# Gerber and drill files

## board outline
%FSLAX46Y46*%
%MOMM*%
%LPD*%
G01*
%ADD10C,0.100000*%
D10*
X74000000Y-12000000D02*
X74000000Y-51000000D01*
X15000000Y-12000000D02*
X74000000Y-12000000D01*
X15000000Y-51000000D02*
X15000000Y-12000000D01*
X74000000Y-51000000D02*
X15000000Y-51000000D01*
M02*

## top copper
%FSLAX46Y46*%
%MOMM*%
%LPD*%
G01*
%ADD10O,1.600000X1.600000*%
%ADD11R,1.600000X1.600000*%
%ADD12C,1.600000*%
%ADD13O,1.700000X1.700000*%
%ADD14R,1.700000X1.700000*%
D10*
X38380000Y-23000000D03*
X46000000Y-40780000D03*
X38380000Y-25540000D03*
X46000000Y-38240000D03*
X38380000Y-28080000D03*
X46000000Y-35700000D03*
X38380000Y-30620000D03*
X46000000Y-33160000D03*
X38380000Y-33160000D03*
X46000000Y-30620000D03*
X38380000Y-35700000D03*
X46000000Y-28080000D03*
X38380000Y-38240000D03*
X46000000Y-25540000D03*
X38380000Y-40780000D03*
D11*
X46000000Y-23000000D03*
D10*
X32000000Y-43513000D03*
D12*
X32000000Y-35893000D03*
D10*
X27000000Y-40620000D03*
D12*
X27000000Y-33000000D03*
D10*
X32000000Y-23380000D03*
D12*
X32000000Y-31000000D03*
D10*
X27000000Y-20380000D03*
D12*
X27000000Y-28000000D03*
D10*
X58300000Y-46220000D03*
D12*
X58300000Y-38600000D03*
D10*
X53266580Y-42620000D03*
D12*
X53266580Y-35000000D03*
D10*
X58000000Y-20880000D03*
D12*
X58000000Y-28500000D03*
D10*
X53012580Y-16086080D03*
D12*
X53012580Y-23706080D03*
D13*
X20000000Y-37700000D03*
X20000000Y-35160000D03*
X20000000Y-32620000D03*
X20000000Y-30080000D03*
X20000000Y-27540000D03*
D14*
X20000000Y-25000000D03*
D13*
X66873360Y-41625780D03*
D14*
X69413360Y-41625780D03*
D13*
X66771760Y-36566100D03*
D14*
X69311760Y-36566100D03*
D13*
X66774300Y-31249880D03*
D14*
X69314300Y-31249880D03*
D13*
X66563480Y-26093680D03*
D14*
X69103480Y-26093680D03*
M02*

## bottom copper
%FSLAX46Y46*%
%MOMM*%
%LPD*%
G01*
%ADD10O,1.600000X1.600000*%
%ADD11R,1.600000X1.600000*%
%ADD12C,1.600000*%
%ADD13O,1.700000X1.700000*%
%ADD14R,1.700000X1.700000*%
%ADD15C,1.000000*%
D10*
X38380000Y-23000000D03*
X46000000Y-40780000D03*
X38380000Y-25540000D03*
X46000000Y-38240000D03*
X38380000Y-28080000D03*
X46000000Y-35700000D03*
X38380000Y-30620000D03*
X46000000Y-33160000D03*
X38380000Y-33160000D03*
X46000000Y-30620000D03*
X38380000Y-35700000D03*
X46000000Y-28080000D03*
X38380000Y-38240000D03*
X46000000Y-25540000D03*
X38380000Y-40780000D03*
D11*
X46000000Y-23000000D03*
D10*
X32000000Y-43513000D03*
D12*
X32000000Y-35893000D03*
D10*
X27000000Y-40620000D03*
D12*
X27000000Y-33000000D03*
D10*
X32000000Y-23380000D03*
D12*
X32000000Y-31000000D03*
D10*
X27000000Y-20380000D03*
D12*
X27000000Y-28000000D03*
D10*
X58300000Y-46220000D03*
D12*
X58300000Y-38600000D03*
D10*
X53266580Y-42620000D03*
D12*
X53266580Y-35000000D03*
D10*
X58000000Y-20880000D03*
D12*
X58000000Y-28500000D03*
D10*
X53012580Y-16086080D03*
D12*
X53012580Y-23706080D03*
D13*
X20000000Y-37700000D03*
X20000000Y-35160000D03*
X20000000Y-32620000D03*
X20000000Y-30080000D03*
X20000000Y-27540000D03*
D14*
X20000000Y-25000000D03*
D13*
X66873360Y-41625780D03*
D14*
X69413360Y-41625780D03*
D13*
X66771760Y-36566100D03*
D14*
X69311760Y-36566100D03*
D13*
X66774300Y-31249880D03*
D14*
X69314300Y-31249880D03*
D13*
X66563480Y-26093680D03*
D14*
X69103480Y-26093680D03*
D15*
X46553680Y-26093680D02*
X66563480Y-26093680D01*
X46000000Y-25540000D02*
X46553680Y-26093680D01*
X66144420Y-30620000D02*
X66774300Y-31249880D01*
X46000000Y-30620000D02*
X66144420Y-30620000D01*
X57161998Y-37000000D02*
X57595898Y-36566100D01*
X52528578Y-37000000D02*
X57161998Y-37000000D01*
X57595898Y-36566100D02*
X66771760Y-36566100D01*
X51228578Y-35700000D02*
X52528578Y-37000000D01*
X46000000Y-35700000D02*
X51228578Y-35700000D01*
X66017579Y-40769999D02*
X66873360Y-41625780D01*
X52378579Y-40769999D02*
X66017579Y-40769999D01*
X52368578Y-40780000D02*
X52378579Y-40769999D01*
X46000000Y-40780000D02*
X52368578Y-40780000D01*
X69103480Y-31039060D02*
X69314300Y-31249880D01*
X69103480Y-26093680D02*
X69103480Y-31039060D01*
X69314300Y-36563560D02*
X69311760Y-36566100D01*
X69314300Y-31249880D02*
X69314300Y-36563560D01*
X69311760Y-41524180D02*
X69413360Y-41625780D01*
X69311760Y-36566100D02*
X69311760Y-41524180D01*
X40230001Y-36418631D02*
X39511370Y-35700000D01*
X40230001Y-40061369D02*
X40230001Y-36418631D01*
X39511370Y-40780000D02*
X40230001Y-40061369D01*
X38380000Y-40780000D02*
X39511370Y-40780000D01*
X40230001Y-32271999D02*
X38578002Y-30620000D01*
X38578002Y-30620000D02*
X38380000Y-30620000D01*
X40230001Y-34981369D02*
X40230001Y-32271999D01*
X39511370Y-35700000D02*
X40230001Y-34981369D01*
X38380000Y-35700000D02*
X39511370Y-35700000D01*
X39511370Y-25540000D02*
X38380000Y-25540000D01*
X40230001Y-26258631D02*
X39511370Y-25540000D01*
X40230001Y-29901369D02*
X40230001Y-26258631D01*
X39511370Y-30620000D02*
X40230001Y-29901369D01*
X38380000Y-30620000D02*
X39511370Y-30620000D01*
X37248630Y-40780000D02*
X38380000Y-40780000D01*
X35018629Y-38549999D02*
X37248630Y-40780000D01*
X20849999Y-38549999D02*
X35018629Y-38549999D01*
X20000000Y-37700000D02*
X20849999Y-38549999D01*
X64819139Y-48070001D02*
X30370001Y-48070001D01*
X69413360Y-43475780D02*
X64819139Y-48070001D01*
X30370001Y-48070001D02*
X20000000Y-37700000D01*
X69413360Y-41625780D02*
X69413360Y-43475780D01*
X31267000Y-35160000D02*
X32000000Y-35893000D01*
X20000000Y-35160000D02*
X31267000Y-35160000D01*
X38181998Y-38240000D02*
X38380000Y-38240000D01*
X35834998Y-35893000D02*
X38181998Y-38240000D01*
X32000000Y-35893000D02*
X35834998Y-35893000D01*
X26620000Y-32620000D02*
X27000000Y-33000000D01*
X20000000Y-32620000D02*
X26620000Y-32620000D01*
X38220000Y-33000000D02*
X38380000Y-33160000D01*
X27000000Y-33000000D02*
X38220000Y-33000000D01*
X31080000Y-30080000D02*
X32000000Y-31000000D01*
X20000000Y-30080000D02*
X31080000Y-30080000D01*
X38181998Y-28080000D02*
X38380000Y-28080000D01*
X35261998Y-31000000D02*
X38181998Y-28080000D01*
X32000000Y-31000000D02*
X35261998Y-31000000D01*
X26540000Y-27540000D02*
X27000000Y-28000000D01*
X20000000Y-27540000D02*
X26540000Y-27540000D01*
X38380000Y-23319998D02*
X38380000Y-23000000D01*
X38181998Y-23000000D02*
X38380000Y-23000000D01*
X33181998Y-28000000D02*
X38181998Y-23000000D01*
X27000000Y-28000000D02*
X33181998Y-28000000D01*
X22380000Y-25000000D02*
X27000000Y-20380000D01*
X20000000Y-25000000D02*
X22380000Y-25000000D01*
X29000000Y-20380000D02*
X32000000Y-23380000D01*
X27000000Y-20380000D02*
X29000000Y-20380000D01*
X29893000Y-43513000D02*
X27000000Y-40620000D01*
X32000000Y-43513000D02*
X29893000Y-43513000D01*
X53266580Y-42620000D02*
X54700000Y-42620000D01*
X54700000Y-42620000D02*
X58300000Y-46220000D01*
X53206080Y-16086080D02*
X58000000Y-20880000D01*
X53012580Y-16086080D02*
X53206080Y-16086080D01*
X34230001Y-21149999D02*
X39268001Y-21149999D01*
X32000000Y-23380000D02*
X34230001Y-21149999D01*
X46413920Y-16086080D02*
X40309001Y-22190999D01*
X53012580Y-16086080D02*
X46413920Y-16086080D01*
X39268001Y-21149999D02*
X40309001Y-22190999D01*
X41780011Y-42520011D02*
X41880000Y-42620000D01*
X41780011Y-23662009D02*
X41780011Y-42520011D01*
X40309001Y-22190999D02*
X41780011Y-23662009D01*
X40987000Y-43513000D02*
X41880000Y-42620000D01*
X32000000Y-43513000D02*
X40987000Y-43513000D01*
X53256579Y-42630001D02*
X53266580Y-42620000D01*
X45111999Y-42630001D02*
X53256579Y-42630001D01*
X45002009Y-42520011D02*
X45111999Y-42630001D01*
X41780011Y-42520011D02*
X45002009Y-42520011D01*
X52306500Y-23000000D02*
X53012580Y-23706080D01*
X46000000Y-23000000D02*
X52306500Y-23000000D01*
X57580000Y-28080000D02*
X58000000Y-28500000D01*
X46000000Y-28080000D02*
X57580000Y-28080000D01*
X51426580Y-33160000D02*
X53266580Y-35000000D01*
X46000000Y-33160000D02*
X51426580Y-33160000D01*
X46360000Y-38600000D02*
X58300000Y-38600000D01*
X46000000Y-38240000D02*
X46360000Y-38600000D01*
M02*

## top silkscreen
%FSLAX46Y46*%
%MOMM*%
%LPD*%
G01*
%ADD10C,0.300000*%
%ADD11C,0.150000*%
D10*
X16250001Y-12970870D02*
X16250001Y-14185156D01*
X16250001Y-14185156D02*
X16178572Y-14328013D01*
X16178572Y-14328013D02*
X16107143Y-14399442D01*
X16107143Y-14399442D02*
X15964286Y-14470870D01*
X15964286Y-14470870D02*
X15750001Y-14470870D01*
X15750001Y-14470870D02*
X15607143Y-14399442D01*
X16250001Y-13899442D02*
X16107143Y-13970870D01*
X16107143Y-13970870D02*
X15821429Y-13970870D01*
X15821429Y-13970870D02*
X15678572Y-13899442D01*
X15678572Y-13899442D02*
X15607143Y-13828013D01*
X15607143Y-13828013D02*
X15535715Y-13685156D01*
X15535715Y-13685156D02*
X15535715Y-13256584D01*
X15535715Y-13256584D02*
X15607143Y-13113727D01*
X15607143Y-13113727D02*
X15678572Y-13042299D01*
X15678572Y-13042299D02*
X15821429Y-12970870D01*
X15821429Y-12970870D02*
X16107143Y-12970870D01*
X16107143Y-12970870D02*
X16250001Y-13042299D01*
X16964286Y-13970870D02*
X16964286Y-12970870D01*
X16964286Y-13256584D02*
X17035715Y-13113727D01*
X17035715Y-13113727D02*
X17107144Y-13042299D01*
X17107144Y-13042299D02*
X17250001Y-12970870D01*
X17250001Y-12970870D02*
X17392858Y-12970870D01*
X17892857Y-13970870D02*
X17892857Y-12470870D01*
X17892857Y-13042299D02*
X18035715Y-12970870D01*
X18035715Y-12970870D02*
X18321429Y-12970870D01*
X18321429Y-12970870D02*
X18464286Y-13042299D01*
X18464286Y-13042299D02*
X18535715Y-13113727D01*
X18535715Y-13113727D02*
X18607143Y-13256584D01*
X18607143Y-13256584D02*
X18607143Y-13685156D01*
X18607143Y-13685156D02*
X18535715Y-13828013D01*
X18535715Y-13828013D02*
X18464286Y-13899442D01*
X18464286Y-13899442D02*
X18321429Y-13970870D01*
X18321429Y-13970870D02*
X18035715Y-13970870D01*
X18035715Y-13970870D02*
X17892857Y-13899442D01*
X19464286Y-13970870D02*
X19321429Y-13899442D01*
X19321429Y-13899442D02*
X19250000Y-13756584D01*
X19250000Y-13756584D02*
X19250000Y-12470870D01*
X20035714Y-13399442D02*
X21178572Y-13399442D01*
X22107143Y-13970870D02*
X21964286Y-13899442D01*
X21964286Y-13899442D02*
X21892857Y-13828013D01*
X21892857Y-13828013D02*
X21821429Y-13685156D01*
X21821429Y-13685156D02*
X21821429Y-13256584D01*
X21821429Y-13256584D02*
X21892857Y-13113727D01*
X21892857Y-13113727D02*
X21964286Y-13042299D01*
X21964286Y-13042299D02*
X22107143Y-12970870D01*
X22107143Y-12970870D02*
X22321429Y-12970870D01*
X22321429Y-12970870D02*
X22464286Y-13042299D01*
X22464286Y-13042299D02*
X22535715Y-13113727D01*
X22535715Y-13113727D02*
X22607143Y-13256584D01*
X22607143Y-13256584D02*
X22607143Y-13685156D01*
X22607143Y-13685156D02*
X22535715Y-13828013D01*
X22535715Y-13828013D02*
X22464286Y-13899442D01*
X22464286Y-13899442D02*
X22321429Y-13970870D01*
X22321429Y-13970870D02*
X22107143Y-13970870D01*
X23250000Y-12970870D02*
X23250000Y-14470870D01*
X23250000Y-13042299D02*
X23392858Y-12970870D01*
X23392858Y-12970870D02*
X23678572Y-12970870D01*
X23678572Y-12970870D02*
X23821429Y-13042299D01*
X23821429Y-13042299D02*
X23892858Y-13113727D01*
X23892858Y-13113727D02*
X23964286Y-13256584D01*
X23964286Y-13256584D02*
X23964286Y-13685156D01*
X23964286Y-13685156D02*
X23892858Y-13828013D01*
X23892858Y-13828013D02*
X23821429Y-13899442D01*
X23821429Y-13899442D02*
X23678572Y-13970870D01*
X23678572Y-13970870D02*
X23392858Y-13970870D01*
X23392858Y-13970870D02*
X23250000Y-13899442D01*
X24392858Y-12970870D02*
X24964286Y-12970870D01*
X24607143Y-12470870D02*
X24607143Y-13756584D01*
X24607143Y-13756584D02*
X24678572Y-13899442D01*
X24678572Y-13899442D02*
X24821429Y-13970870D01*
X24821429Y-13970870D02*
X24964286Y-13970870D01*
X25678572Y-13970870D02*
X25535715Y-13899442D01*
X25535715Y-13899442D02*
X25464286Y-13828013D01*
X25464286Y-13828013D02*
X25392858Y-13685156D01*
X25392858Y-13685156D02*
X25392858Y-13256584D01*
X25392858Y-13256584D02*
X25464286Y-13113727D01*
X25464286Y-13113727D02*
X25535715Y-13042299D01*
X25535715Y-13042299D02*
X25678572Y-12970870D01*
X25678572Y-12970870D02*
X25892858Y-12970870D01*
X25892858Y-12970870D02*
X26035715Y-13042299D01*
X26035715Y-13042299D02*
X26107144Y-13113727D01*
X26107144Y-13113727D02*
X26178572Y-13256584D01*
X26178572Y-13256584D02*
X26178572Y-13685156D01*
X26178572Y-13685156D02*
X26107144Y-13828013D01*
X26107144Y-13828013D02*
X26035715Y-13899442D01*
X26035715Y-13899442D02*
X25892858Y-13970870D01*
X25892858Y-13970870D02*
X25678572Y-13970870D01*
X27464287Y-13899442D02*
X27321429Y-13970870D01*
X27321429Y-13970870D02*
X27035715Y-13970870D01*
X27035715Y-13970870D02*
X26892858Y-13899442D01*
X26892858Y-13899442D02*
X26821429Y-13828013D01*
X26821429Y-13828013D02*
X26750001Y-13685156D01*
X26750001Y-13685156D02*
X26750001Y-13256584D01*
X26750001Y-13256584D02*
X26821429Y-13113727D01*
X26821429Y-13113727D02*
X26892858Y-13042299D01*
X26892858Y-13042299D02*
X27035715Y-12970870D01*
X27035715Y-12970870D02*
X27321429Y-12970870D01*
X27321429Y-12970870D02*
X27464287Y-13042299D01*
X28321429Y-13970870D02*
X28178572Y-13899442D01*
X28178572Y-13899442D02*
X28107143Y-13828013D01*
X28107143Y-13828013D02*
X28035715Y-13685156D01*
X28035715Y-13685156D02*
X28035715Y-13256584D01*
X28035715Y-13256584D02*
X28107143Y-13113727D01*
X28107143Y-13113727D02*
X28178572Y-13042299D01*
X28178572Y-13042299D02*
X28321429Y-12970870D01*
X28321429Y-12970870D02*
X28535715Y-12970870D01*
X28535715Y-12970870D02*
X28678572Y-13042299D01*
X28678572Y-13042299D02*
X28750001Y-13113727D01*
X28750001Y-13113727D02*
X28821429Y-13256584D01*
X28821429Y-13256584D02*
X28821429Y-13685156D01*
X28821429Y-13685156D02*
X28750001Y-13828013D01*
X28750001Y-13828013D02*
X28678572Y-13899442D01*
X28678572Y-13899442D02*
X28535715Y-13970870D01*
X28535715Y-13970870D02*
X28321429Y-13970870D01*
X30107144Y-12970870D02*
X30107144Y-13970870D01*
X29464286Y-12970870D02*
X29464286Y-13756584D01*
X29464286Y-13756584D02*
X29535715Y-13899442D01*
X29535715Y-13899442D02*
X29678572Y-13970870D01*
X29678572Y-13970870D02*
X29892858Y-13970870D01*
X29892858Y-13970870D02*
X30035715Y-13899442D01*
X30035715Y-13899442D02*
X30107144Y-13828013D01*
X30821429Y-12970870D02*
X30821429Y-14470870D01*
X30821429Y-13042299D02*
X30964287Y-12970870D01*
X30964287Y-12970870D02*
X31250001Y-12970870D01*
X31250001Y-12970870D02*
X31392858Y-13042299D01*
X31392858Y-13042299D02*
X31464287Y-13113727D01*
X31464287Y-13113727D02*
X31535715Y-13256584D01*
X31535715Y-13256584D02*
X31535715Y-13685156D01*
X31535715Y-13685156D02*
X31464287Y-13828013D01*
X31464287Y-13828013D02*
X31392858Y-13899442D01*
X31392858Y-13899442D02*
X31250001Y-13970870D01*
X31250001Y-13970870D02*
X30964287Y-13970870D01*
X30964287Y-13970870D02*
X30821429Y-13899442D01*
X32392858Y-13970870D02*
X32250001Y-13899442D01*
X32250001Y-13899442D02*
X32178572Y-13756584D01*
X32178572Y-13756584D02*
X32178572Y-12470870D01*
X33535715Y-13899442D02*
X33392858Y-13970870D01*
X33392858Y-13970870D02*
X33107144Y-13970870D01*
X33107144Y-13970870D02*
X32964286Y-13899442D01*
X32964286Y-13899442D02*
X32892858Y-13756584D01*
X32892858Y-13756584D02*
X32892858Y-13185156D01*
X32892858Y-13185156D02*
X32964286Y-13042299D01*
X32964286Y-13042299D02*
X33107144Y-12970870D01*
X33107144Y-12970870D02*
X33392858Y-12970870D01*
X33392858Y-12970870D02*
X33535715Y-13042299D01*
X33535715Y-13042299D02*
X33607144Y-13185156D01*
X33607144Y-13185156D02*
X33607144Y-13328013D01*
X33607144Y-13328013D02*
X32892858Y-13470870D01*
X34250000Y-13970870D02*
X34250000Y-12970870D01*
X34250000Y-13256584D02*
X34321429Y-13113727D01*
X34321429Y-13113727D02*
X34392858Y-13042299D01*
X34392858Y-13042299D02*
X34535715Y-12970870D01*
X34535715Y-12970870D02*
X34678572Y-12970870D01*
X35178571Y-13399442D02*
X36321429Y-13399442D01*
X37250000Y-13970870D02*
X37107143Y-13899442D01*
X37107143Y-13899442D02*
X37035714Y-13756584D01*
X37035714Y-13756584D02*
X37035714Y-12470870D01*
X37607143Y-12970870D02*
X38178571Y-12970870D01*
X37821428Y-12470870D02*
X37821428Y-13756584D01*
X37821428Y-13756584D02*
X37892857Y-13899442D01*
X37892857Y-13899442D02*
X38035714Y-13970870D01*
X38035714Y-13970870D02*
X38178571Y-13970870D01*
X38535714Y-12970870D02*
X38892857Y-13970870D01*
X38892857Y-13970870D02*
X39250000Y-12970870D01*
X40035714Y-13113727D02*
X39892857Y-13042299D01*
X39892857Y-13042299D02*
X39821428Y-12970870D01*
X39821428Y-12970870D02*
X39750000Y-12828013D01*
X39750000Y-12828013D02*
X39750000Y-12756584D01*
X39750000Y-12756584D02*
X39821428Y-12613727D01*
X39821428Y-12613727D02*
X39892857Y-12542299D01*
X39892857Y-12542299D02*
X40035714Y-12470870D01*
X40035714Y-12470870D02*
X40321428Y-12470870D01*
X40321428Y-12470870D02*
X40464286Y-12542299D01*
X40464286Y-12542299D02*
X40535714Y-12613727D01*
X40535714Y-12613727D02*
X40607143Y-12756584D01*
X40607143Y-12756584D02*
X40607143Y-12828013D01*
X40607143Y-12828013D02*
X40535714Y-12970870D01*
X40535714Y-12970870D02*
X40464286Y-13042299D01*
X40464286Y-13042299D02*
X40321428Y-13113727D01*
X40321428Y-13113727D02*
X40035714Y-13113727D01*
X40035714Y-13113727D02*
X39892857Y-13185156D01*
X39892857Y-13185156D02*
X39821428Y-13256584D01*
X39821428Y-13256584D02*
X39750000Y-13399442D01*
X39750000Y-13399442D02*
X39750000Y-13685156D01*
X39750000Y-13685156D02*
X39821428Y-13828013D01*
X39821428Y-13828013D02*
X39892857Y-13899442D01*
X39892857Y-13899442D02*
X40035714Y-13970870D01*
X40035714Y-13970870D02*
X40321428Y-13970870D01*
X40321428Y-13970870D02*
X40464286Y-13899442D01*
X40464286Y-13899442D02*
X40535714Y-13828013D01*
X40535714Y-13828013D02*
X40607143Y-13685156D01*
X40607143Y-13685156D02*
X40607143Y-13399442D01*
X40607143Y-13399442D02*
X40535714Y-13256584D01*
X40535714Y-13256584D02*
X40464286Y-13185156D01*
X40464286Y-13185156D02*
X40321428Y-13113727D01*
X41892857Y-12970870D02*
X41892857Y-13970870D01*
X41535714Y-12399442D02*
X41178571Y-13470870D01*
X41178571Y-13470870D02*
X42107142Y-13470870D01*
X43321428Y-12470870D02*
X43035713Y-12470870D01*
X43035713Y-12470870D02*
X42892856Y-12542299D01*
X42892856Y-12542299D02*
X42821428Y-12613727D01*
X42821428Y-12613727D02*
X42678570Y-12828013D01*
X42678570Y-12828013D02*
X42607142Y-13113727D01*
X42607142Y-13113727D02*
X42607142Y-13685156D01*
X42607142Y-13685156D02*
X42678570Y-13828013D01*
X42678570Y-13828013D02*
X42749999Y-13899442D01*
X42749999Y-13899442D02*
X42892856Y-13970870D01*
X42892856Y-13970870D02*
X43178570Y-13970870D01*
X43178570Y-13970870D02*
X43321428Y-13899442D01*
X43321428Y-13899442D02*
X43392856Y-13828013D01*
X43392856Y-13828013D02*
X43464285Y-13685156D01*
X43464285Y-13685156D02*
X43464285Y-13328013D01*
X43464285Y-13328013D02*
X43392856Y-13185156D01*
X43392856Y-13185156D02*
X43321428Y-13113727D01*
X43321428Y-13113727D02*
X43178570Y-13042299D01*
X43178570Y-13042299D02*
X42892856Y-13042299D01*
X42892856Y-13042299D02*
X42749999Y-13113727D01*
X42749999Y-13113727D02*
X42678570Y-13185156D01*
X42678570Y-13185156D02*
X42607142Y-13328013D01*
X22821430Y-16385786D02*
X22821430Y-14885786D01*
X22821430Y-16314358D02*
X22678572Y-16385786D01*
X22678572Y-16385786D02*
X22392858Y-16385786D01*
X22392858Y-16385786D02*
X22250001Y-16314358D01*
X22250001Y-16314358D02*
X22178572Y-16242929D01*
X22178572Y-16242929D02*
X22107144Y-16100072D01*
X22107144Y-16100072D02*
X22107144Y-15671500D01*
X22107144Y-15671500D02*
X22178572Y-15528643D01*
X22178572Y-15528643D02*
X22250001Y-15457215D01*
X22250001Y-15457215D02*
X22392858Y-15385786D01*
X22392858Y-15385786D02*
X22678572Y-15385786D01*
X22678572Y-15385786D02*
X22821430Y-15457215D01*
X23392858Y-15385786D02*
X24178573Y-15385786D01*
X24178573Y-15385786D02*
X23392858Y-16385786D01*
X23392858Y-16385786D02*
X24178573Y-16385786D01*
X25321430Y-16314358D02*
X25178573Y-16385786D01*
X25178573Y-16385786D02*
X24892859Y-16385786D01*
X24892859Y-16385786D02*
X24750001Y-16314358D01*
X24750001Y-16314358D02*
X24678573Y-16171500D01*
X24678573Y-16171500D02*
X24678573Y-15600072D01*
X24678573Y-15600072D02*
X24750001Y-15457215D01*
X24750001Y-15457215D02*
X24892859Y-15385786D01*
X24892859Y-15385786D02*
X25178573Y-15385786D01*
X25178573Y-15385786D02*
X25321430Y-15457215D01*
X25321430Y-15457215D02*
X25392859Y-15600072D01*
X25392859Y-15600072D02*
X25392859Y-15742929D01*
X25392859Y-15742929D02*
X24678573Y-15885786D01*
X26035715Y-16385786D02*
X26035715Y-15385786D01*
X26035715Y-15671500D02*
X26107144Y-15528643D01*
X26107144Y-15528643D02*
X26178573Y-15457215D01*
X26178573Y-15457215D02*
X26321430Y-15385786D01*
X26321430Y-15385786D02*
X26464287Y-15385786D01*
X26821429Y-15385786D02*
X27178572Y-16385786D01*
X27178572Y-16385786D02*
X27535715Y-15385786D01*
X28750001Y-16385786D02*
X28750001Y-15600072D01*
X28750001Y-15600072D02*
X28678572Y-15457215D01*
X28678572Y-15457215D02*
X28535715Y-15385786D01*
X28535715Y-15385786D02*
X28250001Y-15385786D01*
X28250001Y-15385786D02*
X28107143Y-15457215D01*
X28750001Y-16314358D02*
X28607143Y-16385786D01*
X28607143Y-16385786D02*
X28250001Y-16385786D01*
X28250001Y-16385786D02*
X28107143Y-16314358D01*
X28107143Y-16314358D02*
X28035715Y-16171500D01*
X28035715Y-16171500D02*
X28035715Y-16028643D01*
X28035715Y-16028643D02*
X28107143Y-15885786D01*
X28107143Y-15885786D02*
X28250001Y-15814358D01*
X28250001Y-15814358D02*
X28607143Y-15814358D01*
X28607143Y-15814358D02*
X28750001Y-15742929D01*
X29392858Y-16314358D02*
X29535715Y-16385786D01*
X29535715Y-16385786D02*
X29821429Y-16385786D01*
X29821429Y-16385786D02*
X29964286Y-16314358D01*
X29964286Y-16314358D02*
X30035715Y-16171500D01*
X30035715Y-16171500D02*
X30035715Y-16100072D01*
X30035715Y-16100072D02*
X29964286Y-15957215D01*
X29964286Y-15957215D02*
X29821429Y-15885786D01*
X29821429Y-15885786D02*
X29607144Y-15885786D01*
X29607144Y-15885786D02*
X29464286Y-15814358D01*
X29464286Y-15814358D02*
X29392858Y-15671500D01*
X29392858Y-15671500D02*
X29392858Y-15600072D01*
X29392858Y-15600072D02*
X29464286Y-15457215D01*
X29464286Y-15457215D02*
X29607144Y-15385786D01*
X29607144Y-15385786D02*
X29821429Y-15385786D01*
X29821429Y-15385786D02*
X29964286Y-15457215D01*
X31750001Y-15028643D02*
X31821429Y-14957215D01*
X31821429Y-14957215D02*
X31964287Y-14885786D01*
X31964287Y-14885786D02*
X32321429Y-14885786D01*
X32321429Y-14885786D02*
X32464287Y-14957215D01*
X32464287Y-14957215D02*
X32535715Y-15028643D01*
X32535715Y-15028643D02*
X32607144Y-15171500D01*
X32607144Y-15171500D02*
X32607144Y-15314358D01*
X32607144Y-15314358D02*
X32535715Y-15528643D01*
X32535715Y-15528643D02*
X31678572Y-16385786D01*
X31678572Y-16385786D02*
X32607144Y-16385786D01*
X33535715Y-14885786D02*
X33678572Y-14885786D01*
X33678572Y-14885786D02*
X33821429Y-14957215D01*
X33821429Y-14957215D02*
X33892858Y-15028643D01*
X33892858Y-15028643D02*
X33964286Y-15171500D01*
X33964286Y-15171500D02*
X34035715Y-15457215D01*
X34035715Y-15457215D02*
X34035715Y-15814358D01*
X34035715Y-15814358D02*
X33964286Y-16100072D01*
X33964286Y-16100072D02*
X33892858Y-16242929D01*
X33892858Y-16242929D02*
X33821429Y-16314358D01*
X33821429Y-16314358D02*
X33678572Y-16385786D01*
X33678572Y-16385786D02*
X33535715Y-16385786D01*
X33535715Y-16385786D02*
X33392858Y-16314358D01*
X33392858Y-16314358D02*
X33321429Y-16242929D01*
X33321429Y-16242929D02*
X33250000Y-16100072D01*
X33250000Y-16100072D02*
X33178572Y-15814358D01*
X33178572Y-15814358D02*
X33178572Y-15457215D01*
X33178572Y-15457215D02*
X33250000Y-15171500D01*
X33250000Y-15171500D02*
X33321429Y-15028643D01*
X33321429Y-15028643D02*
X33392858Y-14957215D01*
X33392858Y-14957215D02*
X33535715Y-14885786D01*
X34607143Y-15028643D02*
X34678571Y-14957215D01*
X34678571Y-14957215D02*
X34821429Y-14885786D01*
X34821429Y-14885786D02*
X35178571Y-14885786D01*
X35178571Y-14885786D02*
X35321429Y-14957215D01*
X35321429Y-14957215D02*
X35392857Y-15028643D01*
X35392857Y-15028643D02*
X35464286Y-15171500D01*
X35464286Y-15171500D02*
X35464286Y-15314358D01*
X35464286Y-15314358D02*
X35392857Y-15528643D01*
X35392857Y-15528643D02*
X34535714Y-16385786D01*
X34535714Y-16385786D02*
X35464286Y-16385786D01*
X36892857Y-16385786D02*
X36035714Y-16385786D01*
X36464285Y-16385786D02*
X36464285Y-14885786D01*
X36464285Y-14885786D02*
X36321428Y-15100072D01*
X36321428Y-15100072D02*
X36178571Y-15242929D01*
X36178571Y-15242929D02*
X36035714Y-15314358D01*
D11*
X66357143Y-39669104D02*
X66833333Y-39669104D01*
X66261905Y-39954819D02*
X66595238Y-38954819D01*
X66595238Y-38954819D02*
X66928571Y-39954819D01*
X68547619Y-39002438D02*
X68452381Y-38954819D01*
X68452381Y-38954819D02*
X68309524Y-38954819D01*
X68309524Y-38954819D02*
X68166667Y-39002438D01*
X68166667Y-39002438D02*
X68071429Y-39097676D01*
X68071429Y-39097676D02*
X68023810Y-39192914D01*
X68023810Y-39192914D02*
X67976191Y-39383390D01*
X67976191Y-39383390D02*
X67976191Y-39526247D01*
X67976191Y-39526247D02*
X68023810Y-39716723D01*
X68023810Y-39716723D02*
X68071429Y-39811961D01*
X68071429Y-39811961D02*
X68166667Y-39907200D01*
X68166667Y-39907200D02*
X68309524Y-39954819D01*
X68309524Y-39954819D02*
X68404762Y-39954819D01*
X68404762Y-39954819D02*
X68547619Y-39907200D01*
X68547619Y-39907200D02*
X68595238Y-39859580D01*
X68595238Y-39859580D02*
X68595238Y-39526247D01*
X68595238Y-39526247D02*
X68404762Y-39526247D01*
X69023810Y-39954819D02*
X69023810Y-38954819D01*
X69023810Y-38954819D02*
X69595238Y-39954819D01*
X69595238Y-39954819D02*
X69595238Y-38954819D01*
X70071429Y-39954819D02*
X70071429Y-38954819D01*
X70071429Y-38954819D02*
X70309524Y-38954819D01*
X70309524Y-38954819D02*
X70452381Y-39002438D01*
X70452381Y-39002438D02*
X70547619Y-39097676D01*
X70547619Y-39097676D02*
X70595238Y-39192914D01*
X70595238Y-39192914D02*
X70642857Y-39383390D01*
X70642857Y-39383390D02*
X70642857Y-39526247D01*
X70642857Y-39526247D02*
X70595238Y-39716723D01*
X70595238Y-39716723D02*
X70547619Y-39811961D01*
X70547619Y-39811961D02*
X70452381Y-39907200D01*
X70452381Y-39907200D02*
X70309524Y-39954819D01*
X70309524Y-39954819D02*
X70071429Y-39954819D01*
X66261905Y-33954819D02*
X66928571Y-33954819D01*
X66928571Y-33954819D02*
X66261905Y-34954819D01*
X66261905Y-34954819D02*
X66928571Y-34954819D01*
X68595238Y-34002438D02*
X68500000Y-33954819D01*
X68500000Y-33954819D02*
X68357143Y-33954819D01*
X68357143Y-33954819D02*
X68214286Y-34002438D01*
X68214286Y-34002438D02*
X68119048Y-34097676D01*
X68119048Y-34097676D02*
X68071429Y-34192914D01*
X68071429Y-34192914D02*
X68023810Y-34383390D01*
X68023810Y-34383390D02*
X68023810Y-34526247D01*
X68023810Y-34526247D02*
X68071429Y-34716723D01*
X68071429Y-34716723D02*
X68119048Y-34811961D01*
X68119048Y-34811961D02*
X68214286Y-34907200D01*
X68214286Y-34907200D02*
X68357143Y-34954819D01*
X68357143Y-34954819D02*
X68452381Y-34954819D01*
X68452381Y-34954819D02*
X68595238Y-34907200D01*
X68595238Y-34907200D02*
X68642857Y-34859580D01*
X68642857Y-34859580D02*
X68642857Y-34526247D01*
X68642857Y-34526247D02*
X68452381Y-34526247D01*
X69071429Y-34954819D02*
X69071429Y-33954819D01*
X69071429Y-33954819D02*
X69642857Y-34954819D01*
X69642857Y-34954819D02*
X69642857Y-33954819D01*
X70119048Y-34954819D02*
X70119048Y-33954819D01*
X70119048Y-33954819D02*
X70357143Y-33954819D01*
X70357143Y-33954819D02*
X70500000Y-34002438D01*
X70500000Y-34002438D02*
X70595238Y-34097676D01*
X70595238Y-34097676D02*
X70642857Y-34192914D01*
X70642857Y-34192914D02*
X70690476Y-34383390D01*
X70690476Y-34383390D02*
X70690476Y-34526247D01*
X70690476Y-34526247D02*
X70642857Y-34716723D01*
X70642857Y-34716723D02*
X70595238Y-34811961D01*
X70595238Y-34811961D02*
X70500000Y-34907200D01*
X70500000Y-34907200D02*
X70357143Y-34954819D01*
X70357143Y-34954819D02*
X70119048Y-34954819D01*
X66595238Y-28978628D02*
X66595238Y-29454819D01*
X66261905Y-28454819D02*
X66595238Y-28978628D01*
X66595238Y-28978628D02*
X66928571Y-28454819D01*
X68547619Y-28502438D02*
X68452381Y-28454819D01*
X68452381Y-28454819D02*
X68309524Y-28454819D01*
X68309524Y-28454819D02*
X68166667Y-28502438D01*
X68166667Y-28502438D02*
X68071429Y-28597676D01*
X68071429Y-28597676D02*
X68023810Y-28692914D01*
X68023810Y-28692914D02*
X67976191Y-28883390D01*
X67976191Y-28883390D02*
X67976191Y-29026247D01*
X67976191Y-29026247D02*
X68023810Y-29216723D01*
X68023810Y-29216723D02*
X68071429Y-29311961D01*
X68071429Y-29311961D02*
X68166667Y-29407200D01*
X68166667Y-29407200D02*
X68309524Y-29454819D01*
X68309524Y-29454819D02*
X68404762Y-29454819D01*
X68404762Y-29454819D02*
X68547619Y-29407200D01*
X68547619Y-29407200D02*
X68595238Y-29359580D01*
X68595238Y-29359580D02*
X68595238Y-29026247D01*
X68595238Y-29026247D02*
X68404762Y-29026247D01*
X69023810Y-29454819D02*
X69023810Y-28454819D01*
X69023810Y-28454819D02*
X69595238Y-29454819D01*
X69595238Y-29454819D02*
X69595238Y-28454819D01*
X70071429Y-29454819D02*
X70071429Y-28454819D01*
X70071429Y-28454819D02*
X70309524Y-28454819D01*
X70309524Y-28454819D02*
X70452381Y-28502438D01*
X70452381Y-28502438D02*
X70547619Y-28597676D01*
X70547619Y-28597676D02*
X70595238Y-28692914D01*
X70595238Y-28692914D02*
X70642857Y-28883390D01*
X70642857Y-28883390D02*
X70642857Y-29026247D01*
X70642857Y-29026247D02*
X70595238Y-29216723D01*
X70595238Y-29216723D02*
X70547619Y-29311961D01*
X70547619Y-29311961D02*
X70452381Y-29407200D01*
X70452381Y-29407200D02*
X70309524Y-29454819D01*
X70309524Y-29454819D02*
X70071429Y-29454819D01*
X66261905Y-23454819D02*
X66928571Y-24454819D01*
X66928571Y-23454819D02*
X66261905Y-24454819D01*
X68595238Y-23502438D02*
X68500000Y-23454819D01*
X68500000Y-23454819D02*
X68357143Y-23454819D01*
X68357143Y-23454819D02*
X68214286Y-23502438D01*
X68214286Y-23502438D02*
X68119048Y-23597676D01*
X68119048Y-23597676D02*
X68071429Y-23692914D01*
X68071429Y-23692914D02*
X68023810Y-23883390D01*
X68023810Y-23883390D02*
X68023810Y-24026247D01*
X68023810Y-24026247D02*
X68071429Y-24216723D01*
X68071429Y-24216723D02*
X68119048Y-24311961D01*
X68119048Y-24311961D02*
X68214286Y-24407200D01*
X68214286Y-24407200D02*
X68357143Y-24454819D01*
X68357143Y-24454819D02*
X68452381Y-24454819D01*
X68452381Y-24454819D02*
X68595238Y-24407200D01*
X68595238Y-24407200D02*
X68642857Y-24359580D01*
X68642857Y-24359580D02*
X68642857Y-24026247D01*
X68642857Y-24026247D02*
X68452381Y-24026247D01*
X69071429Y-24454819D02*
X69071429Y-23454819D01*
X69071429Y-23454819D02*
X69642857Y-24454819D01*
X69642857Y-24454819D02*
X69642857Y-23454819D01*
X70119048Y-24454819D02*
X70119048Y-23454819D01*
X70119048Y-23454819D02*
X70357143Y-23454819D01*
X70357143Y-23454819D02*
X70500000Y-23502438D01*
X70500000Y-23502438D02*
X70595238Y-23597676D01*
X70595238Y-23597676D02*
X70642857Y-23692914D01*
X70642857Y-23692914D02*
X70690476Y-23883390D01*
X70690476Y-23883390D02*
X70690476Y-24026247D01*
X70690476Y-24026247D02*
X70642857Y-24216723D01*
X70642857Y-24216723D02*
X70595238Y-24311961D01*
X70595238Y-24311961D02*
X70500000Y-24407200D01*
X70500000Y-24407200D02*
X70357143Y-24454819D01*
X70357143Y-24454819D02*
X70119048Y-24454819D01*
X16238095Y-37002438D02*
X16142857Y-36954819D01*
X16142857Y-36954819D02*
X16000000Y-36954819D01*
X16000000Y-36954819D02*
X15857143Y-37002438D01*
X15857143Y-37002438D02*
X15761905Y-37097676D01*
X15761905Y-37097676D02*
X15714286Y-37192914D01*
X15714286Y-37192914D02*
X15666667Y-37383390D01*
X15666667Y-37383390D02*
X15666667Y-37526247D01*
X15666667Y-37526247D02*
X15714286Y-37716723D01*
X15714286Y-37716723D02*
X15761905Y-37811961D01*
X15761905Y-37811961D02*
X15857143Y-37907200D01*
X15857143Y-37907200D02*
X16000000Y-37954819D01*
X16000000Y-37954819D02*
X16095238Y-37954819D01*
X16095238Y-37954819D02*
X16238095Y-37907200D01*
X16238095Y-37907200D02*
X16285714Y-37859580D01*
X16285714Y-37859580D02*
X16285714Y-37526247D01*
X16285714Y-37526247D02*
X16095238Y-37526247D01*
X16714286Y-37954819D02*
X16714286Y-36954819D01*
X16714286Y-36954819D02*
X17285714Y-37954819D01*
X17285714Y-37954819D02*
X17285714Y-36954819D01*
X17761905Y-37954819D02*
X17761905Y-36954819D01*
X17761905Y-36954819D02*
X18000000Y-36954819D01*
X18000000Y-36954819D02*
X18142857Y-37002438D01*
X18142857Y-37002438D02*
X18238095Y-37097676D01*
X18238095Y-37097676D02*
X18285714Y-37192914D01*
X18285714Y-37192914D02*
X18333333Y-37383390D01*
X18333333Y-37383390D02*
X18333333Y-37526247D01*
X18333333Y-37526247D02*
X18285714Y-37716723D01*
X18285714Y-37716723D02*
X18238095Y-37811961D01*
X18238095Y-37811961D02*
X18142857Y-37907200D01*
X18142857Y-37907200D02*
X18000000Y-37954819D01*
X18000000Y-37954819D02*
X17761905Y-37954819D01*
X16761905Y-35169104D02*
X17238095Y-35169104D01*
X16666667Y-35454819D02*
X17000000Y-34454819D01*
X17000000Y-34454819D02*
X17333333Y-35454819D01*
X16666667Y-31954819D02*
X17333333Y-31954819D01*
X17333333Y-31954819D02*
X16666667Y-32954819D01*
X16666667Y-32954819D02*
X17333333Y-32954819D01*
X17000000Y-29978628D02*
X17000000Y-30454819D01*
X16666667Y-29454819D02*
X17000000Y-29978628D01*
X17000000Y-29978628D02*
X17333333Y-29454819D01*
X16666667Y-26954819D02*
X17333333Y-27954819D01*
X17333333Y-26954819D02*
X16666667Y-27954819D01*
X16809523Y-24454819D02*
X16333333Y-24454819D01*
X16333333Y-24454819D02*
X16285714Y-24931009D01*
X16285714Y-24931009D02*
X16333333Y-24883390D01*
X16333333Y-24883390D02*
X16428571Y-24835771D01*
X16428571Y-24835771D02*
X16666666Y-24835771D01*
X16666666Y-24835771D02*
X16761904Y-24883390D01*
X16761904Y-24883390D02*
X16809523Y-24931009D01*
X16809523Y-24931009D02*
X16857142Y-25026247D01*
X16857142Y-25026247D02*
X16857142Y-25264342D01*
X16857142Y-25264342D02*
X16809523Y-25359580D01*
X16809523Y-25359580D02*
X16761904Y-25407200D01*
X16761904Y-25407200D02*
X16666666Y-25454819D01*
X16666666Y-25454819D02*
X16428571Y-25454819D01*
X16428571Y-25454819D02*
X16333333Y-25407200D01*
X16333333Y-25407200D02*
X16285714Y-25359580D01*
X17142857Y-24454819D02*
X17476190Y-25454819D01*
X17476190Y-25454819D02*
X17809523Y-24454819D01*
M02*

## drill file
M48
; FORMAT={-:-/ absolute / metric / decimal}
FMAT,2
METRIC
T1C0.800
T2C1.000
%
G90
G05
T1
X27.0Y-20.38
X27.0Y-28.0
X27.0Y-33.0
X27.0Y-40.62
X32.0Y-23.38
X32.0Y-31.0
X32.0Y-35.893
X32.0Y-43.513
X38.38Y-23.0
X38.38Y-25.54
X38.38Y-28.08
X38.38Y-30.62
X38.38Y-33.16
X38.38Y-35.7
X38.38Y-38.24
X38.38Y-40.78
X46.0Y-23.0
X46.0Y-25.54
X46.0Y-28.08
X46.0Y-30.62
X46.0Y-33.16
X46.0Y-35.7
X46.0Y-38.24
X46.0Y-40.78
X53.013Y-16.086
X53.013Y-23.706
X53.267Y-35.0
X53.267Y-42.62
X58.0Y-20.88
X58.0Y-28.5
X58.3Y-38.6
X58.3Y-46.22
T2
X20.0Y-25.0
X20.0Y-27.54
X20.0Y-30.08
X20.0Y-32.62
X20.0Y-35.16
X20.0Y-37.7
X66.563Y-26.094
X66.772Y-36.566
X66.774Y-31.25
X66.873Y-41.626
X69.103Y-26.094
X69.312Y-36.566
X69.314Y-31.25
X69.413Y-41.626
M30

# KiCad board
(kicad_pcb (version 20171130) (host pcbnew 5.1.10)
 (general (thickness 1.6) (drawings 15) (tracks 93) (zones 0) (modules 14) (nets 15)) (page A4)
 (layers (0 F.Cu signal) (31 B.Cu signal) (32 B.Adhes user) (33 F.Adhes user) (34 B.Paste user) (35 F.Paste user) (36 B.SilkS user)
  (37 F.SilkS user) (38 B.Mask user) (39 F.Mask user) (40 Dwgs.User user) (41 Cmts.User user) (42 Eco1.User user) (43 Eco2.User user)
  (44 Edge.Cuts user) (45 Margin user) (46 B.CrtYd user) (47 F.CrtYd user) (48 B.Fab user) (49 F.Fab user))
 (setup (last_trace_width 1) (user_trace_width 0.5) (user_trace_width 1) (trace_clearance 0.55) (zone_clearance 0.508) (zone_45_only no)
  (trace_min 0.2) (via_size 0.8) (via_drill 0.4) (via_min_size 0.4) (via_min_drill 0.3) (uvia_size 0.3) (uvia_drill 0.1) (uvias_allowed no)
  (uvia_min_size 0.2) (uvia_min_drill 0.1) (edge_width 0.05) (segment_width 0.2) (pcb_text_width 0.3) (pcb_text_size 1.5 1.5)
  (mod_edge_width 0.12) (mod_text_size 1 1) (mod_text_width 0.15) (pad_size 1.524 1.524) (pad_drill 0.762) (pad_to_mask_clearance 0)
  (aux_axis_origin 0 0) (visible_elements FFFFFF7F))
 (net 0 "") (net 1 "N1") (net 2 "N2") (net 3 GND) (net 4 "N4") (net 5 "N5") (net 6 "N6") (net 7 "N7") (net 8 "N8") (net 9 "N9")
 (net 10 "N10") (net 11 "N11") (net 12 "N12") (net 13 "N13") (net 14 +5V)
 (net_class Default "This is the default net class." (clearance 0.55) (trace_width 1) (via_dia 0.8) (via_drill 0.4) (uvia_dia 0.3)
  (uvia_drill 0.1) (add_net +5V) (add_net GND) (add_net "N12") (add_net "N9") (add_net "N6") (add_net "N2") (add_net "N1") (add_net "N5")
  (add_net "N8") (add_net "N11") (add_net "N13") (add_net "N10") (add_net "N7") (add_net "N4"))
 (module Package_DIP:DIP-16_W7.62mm (layer B.Cu) (at 46 23 180)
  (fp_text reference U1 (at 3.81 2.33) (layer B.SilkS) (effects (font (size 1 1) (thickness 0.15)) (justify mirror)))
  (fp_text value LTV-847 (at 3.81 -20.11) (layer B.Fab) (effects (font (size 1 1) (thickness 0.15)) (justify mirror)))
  (pad 16 thru_hole oval (at 7.62 0 180) (size 1.6 1.6) (drill 0.8) (layers *.Cu *.Mask) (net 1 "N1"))
  (pad 8 thru_hole oval (at 0 -17.78 180) (size 1.6 1.6) (drill 0.8) (layers *.Cu *.Mask) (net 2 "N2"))
  (pad 15 thru_hole oval (at 7.62 -2.54 180) (size 1.6 1.6) (drill 0.8) (layers *.Cu *.Mask) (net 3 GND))
  (pad 7 thru_hole oval (at 0 -15.24 180) (size 1.6 1.6) (drill 0.8) (layers *.Cu *.Mask) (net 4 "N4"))
  (pad 14 thru_hole oval (at 7.62 -5.08 180) (size 1.6 1.6) (drill 0.8) (layers *.Cu *.Mask) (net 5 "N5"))
  (pad 6 thru_hole oval (at 0 -12.7 180) (size 1.6 1.6) (drill 0.8) (layers *.Cu *.Mask) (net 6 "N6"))
  (pad 13 thru_hole oval (at 7.62 -7.62 180) (size 1.6 1.6) (drill 0.8) (layers *.Cu *.Mask) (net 3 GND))
  (pad 5 thru_hole oval (at 0 -10.16 180) (size 1.6 1.6) (drill 0.8) (layers *.Cu *.Mask) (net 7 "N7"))
  (pad 12 thru_hole oval (at 7.62 -10.16 180) (size 1.6 1.6) (drill 0.8) (layers *.Cu *.Mask) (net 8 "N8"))
  (pad 4 thru_hole oval (at 0 -7.62 180) (size 1.6 1.6) (drill 0.8) (layers *.Cu *.Mask) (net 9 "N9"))
  (pad 11 thru_hole oval (at 7.62 -12.7 180) (size 1.6 1.6) (drill 0.8) (layers *.Cu *.Mask) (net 3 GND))
  (pad 3 thru_hole oval (at 0 -5.08 180) (size 1.6 1.6) (drill 0.8) (layers *.Cu *.Mask) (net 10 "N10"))
  (pad 10 thru_hole oval (at 7.62 -15.24 180) (size 1.6 1.6) (drill 0.8) (layers *.Cu *.Mask) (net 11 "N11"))
  (pad 2 thru_hole oval (at 0 -2.54 180) (size 1.6 1.6) (drill 0.8) (layers *.Cu *.Mask) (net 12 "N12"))
  (pad 9 thru_hole oval (at 7.62 -17.78 180) (size 1.6 1.6) (drill 0.8) (layers *.Cu *.Mask) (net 3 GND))
  (pad 1 thru_hole rect (at 0 0 180) (size 1.6 1.6) (drill 0.8) (layers *.Cu *.Mask) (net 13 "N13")))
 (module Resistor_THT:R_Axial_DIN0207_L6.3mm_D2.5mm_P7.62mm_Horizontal (layer B.Cu) (at 32 35.893 270)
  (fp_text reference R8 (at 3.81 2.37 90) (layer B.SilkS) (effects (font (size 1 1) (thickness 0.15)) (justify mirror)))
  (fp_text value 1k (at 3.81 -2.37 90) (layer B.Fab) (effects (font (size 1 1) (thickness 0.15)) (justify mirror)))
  (pad 2 thru_hole oval (at 7.62 0 270) (size 1.6 1.6) (drill 0.8) (layers *.Cu *.Mask) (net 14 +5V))
  (pad 1 thru_hole circle (at 0 0 270) (size 1.6 1.6) (drill 0.8) (layers *.Cu *.Mask) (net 11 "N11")))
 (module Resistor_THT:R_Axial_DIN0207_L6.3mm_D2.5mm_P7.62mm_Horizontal (layer B.Cu) (at 27 33 270)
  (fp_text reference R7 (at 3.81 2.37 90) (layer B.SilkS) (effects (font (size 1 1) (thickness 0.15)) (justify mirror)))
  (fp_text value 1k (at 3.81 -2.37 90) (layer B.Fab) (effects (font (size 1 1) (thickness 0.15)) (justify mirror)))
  (pad 2 thru_hole oval (at 7.62 0 270) (size 1.6 1.6) (drill 0.8) (layers *.Cu *.Mask) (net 14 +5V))
  (pad 1 thru_hole circle (at 0 0 270) (size 1.6 1.6) (drill 0.8) (layers *.Cu *.Mask) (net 8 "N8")))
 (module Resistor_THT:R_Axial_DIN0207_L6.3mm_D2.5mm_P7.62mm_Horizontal (layer B.Cu) (at 32 31 90)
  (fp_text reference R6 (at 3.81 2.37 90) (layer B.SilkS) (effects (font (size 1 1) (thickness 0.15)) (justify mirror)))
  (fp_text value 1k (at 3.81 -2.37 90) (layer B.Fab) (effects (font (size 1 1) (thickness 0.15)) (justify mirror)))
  (pad 2 thru_hole oval (at 7.62 0 90) (size 1.6 1.6) (drill 0.8) (layers *.Cu *.Mask) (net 14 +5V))
  (pad 1 thru_hole circle (at 0 0 90) (size 1.6 1.6) (drill 0.8) (layers *.Cu *.Mask) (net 5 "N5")))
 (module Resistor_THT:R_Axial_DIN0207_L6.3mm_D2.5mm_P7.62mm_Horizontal (layer B.Cu) (at 27 28 90)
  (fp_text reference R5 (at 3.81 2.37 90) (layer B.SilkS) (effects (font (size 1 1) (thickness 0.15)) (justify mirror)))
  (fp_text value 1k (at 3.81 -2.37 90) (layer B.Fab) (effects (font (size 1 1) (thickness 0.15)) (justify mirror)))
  (pad 2 thru_hole oval (at 7.62 0 90) (size 1.6 1.6) (drill 0.8) (layers *.Cu *.Mask) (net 14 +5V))
  (pad 1 thru_hole circle (at 0 0 90) (size 1.6 1.6) (drill 0.8) (layers *.Cu *.Mask) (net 1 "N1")))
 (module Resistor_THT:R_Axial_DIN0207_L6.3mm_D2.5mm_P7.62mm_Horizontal (layer B.Cu) (at 58.3 38.6 270)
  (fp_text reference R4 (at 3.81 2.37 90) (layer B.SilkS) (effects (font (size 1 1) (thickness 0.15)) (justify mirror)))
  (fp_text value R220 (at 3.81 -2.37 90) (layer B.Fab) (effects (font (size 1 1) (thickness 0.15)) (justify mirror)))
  (pad 2 thru_hole oval (at 7.62 0 270) (size 1.6 1.6) (drill 0.8) (layers *.Cu *.Mask) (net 14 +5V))
  (pad 1 thru_hole circle (at 0 0 270) (size 1.6 1.6) (drill 0.8) (layers *.Cu *.Mask) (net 4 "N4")))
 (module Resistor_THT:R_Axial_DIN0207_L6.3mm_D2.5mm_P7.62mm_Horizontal (layer B.Cu) (at 53.26658 35 270)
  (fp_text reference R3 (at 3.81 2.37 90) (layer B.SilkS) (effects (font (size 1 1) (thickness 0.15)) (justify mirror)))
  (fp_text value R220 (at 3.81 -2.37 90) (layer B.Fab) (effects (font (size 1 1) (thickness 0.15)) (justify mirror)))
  (pad 2 thru_hole oval (at 7.62 0 270) (size 1.6 1.6) (drill 0.8) (layers *.Cu *.Mask) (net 14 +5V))
  (pad 1 thru_hole circle (at 0 0 270) (size 1.6 1.6) (drill 0.8) (layers *.Cu *.Mask) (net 7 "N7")))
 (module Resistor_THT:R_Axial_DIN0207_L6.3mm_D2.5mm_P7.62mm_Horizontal (layer B.Cu) (at 58 28.5 90)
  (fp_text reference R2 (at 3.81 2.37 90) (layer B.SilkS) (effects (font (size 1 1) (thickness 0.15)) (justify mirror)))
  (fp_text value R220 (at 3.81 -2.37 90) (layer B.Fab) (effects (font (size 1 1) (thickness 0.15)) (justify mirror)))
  (pad 2 thru_hole oval (at 7.62 0 90) (size 1.6 1.6) (drill 0.8) (layers *.Cu *.Mask) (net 14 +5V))
  (pad 1 thru_hole circle (at 0 0 90) (size 1.6 1.6) (drill 0.8) (layers *.Cu *.Mask) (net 10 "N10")))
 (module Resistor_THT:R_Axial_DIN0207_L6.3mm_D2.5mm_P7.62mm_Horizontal (layer B.Cu) (at 53.01258 23.70608 90)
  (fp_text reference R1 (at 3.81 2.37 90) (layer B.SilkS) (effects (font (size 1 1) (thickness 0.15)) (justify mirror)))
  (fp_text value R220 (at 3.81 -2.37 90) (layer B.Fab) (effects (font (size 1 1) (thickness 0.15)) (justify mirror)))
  (pad 2 thru_hole oval (at 7.62 0 90) (size 1.6 1.6) (drill 0.8) (layers *.Cu *.Mask) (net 14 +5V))
  (pad 1 thru_hole circle (at 0 0 90) (size 1.6 1.6) (drill 0.8) (layers *.Cu *.Mask) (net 13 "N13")))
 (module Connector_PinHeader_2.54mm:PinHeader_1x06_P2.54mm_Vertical (layer B.Cu) (at 20 25 180)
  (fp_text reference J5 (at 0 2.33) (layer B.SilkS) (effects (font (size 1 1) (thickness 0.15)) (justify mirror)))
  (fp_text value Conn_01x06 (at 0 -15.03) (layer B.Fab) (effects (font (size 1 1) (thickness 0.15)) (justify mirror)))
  (pad 6 thru_hole oval (at 0 -12.7 180) (size 1.7 1.7) (drill 1) (layers *.Cu *.Mask) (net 3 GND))
  (pad 5 thru_hole oval (at 0 -10.16 180) (size 1.7 1.7) (drill 1) (layers *.Cu *.Mask) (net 11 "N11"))
  (pad 4 thru_hole oval (at 0 -7.62 180) (size 1.7 1.7) (drill 1) (layers *.Cu *.Mask) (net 8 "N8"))
  (pad 3 thru_hole oval (at 0 -5.08 180) (size 1.7 1.7) (drill 1) (layers *.Cu *.Mask) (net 5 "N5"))
  (pad 2 thru_hole oval (at 0 -2.54 180) (size 1.7 1.7) (drill 1) (layers *.Cu *.Mask) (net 1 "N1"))
  (pad 1 thru_hole rect (at 0 0 180) (size 1.7 1.7) (drill 1) (layers *.Cu *.Mask) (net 14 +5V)))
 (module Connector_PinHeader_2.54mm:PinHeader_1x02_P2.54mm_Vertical (layer B.Cu) (at 69.41336 41.62578 90)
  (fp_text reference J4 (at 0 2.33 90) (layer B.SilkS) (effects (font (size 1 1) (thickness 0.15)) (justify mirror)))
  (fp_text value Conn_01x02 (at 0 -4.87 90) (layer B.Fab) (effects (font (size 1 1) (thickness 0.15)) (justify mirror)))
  (pad 2 thru_hole oval (at 0 -2.54 90) (size 1.7 1.7) (drill 1) (layers *.Cu *.Mask) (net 2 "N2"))
  (pad 1 thru_hole rect (at 0 0 90) (size 1.7 1.7) (drill 1) (layers *.Cu *.Mask) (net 3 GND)))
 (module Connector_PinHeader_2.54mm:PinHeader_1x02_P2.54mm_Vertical (layer B.Cu) (at 69.31176 36.5661 90)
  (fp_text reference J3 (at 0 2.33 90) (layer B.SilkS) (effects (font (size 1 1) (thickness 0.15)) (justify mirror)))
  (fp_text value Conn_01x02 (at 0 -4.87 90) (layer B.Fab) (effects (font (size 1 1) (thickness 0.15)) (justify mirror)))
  (pad 2 thru_hole oval (at 0 -2.54 90) (size 1.7 1.7) (drill 1) (layers *.Cu *.Mask) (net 6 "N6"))
  (pad 1 thru_hole rect (at 0 0 90) (size 1.7 1.7) (drill 1) (layers *.Cu *.Mask) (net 3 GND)))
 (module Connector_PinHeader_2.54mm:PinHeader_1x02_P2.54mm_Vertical (layer B.Cu) (at 69.3143 31.24988 90)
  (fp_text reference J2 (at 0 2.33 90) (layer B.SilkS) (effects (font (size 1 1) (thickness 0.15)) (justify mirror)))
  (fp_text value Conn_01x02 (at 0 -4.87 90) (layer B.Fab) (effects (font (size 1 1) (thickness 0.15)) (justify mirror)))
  (pad 2 thru_hole oval (at 0 -2.54 90) (size 1.7 1.7) (drill 1) (layers *.Cu *.Mask) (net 9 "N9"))
  (pad 1 thru_hole rect (at 0 0 90) (size 1.7 1.7) (drill 1) (layers *.Cu *.Mask) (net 3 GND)))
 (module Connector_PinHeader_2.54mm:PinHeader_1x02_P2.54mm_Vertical (layer B.Cu) (at 69.10348 26.09368 90)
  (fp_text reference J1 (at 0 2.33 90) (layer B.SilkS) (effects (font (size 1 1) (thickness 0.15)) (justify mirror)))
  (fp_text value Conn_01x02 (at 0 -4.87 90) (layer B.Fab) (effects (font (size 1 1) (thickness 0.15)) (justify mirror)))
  (pad 2 thru_hole oval (at 0 -2.54 90) (size 1.7 1.7) (drill 1) (layers *.Cu *.Mask) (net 12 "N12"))
  (pad 1 thru_hole rect (at 0 0 90) (size 1.7 1.7) (drill 1) (layers *.Cu *.Mask) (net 3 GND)))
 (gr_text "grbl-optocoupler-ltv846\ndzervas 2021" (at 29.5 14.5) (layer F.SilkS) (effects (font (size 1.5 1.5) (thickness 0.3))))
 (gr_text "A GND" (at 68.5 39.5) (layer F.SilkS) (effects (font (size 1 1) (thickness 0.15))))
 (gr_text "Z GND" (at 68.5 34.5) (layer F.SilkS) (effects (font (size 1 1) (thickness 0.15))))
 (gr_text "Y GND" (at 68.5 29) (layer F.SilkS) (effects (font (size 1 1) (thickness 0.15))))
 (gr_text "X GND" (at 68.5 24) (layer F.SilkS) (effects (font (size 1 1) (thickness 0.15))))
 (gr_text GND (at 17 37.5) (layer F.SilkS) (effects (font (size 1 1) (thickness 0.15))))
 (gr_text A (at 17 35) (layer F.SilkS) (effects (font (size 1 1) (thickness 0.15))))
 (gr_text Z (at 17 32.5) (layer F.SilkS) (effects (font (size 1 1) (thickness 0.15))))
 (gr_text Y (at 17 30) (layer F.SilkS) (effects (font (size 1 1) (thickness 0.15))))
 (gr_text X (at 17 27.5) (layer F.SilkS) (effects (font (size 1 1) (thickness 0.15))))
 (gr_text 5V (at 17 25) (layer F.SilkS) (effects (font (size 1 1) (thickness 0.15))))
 (gr_line (start 74 12) (end 74 51) (layer Edge.Cuts) (width 0.1))
 (gr_line (start 15 12) (end 74 12) (layer Edge.Cuts) (width 0.1))
 (gr_line (start 15 51) (end 15 12) (layer Edge.Cuts) (width 0.1))
 (gr_line (start 74 51) (end 15 51) (layer Edge.Cuts) (width 0.1))
 (segment (start 46.55368 26.09368) (end 66.56348 26.09368) (width 1) (layer B.Cu) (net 12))
 (segment (start 46 25.54) (end 46.55368 26.09368) (width 1) (layer B.Cu) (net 12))
 (segment (start 66.14442 30.62) (end 66.7743 31.24988) (width 1) (layer B.Cu) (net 9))
 (segment (start 46 30.62) (end 66.14442 30.62) (width 1) (layer B.Cu) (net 9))
 (segment (start 57.161998 37) (end 57.595898 36.5661) (width 1) (layer B.Cu) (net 6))
 (segment (start 52.528578 37) (end 57.161998 37) (width 1) (layer B.Cu) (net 6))
 (segment (start 57.595898 36.5661) (end 66.77176 36.5661) (width 1) (layer B.Cu) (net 6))
 (segment (start 51.228578 35.7) (end 52.528578 37) (width 1) (layer B.Cu) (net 6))
 (segment (start 46 35.7) (end 51.228578 35.7) (width 1) (layer B.Cu) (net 6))
 (segment (start 66.017579 40.769999) (end 66.87336 41.62578) (width 1) (layer B.Cu) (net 2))
 (segment (start 52.378579 40.769999) (end 66.017579 40.769999) (width 1) (layer B.Cu) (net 2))
 (segment (start 52.368578 40.78) (end 52.378579 40.769999) (width 1) (layer B.Cu) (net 2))
 (segment (start 46 40.78) (end 52.368578 40.78) (width 1) (layer B.Cu) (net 2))
 (segment (start 69.10348 31.03906) (end 69.3143 31.24988) (width 1) (layer B.Cu) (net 3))
 (segment (start 69.10348 26.09368) (end 69.10348 31.03906) (width 1) (layer B.Cu) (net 3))
 (segment (start 69.3143 36.56356) (end 69.31176 36.5661) (width 1) (layer B.Cu) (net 3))
 (segment (start 69.3143 31.24988) (end 69.3143 36.56356) (width 1) (layer B.Cu) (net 3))
 (segment (start 69.31176 41.52418) (end 69.41336 41.62578) (width 1) (layer B.Cu) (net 3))
 (segment (start 69.31176 36.5661) (end 69.31176 41.52418) (width 1) (layer B.Cu) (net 3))
 (segment (start 40.230001 36.418631) (end 39.51137 35.7) (width 1) (layer B.Cu) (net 3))
 (segment (start 40.230001 40.061369) (end 40.230001 36.418631) (width 1) (layer B.Cu) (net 3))
 (segment (start 39.51137 40.78) (end 40.230001 40.061369) (width 1) (layer B.Cu) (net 3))
 (segment (start 38.38 40.78) (end 39.51137 40.78) (width 1) (layer B.Cu) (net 3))
 (segment (start 40.230001 32.271999) (end 38.578002 30.62) (width 1) (layer B.Cu) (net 3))
 (segment (start 38.578002 30.62) (end 38.38 30.62) (width 1) (layer B.Cu) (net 3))
 (segment (start 40.230001 34.981369) (end 40.230001 32.271999) (width 1) (layer B.Cu) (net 3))
 (segment (start 39.51137 35.7) (end 40.230001 34.981369) (width 1) (layer B.Cu) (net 3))
 (segment (start 38.38 35.7) (end 39.51137 35.7) (width 1) (layer B.Cu) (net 3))
 (segment (start 39.51137 25.54) (end 38.38 25.54) (width 1) (layer B.Cu) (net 3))
 (segment (start 40.230001 26.258631) (end 39.51137 25.54) (width 1) (layer B.Cu) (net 3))
 (segment (start 40.230001 29.901369) (end 40.230001 26.258631) (width 1) (layer B.Cu) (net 3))
 (segment (start 39.51137 30.62) (end 40.230001 29.901369) (width 1) (layer B.Cu) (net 3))
 (segment (start 38.38 30.62) (end 39.51137 30.62) (width 1) (layer B.Cu) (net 3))
 (segment (start 37.24863 40.78) (end 38.38 40.78) (width 1) (layer B.Cu) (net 3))
 (segment (start 35.018629 38.549999) (end 37.24863 40.78) (width 1) (layer B.Cu) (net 3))
 (segment (start 20.849999 38.549999) (end 35.018629 38.549999) (width 1) (layer B.Cu) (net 3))
 (segment (start 20 37.7) (end 20.849999 38.549999) (width 1) (layer B.Cu) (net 3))
 (segment (start 64.819139 48.070001) (end 30.370001 48.070001) (width 1) (layer B.Cu) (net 3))
 (segment (start 69.41336 43.47578) (end 64.819139 48.070001) (width 1) (layer B.Cu) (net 3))
 (segment (start 30.370001 48.070001) (end 20 37.7) (width 1) (layer B.Cu) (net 3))
 (segment (start 69.41336 41.62578) (end 69.41336 43.47578) (width 1) (layer B.Cu) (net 3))
 (segment (start 31.267 35.16) (end 32 35.893) (width 1) (layer B.Cu) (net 11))
 (segment (start 20 35.16) (end 31.267 35.16) (width 1) (layer B.Cu) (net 11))
 (segment (start 38.181998 38.24) (end 38.38 38.24) (width 1) (layer B.Cu) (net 11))
 (segment (start 35.834998 35.893) (end 38.181998 38.24) (width 1) (layer B.Cu) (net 11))
 (segment (start 32 35.893) (end 35.834998 35.893) (width 1) (layer B.Cu) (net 11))
 (segment (start 26.62 32.62) (end 27 33) (width 1) (layer B.Cu) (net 8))
 (segment (start 20 32.62) (end 26.62 32.62) (width 1) (layer B.Cu) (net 8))
 (segment (start 38.22 33) (end 38.38 33.16) (width 1) (layer B.Cu) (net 8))
 (segment (start 27 33) (end 38.22 33) (width 1) (layer B.Cu) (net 8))
 (segment (start 31.08 30.08) (end 32 31) (width 1) (layer B.Cu) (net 5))
 (segment (start 20 30.08) (end 31.08 30.08) (width 1) (layer B.Cu) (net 5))
 (segment (start 38.181998 28.08) (end 38.38 28.08) (width 1) (layer B.Cu) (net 5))
 (segment (start 35.261998 31) (end 38.181998 28.08) (width 1) (layer B.Cu) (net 5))
 (segment (start 32 31) (end 35.261998 31) (width 1) (layer B.Cu) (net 5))
 (segment (start 26.54 27.54) (end 27 28) (width 1) (layer B.Cu) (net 1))
 (segment (start 20 27.54) (end 26.54 27.54) (width 1) (layer B.Cu) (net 1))
 (segment (start 38.38 23.319998) (end 38.38 23) (width 1) (layer B.Cu) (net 1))
 (segment (start 38.181998 23) (end 38.38 23) (width 1) (layer B.Cu) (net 1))
 (segment (start 33.181998 28) (end 38.181998 23) (width 1) (layer B.Cu) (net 1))
 (segment (start 27 28) (end 33.181998 28) (width 1) (layer B.Cu) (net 1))
 (segment (start 22.38 25) (end 27 20.38) (width 1) (layer B.Cu) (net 14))
 (segment (start 20 25) (end 22.38 25) (width 1) (layer B.Cu) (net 14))
 (segment (start 29 20.38) (end 32 23.38) (width 1) (layer B.Cu) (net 14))
 (segment (start 27 20.38) (end 29 20.38) (width 1) (layer B.Cu) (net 14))
 (segment (start 29.893 43.513) (end 27 40.62) (width 1) (layer B.Cu) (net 14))
 (segment (start 32 43.513) (end 29.893 43.513) (width 1) (layer B.Cu) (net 14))
 (segment (start 53.26658 42.62) (end 54.7 42.62) (width 1) (layer B.Cu) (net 14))
 (segment (start 54.7 42.62) (end 58.3 46.22) (width 1) (layer B.Cu) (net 14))
 (segment (start 53.20608 16.08608) (end 58 20.88) (width 1) (layer B.Cu) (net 14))
 (segment (start 53.01258 16.08608) (end 53.20608 16.08608) (width 1) (layer B.Cu) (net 14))
 (segment (start 34.230001 21.149999) (end 39.268001 21.149999) (width 1) (layer B.Cu) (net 14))
 (segment (start 32 23.38) (end 34.230001 21.149999) (width 1) (layer B.Cu) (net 14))
 (segment (start 46.41392 16.08608) (end 40.309001 22.190999) (width 1) (layer B.Cu) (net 14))
 (segment (start 53.01258 16.08608) (end 46.41392 16.08608) (width 1) (layer B.Cu) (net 14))
 (segment (start 39.268001 21.149999) (end 40.309001 22.190999) (width 1) (layer B.Cu) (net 14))
 (segment (start 41.780011 42.520011) (end 41.88 42.62) (width 1) (layer B.Cu) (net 14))
 (segment (start 41.780011 23.662009) (end 41.780011 42.520011) (width 1) (layer B.Cu) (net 14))
 (segment (start 40.309001 22.190999) (end 41.780011 23.662009) (width 1) (layer B.Cu) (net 14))
 (segment (start 40.987 43.513) (end 41.88 42.62) (width 1) (layer B.Cu) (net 14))
 (segment (start 32 43.513) (end 40.987 43.513) (width 1) (layer B.Cu) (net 14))
 (segment (start 53.256579 42.630001) (end 53.26658 42.62) (width 1) (layer B.Cu) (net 14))
 (segment (start 45.111999 42.630001) (end 53.256579 42.630001) (width 1) (layer B.Cu) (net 14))
 (segment (start 45.002009 42.520011) (end 45.111999 42.630001) (width 1) (layer B.Cu) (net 14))
 (segment (start 41.780011 42.520011) (end 45.002009 42.520011) (width 1) (layer B.Cu) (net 14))
 (segment (start 52.3065 23) (end 53.01258 23.70608) (width 1) (layer B.Cu) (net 13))
 (segment (start 46 23) (end 52.3065 23) (width 1) (layer B.Cu) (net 13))
 (segment (start 57.58 28.08) (end 58 28.5) (width 1) (layer B.Cu) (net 10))
 (segment (start 46 28.08) (end 57.58 28.08) (width 1) (layer B.Cu) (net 10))
 (segment (start 51.42658 33.16) (end 53.26658 35) (width 1) (layer B.Cu) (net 7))
 (segment (start 46 33.16) (end 51.42658 33.16) (width 1) (layer B.Cu) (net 7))
 (segment (start 46.36 38.6) (end 58.3 38.6) (width 1) (layer B.Cu) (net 4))
 (segment (start 46 38.24) (end 46.36 38.6) (width 1) (layer B.Cu) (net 4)))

